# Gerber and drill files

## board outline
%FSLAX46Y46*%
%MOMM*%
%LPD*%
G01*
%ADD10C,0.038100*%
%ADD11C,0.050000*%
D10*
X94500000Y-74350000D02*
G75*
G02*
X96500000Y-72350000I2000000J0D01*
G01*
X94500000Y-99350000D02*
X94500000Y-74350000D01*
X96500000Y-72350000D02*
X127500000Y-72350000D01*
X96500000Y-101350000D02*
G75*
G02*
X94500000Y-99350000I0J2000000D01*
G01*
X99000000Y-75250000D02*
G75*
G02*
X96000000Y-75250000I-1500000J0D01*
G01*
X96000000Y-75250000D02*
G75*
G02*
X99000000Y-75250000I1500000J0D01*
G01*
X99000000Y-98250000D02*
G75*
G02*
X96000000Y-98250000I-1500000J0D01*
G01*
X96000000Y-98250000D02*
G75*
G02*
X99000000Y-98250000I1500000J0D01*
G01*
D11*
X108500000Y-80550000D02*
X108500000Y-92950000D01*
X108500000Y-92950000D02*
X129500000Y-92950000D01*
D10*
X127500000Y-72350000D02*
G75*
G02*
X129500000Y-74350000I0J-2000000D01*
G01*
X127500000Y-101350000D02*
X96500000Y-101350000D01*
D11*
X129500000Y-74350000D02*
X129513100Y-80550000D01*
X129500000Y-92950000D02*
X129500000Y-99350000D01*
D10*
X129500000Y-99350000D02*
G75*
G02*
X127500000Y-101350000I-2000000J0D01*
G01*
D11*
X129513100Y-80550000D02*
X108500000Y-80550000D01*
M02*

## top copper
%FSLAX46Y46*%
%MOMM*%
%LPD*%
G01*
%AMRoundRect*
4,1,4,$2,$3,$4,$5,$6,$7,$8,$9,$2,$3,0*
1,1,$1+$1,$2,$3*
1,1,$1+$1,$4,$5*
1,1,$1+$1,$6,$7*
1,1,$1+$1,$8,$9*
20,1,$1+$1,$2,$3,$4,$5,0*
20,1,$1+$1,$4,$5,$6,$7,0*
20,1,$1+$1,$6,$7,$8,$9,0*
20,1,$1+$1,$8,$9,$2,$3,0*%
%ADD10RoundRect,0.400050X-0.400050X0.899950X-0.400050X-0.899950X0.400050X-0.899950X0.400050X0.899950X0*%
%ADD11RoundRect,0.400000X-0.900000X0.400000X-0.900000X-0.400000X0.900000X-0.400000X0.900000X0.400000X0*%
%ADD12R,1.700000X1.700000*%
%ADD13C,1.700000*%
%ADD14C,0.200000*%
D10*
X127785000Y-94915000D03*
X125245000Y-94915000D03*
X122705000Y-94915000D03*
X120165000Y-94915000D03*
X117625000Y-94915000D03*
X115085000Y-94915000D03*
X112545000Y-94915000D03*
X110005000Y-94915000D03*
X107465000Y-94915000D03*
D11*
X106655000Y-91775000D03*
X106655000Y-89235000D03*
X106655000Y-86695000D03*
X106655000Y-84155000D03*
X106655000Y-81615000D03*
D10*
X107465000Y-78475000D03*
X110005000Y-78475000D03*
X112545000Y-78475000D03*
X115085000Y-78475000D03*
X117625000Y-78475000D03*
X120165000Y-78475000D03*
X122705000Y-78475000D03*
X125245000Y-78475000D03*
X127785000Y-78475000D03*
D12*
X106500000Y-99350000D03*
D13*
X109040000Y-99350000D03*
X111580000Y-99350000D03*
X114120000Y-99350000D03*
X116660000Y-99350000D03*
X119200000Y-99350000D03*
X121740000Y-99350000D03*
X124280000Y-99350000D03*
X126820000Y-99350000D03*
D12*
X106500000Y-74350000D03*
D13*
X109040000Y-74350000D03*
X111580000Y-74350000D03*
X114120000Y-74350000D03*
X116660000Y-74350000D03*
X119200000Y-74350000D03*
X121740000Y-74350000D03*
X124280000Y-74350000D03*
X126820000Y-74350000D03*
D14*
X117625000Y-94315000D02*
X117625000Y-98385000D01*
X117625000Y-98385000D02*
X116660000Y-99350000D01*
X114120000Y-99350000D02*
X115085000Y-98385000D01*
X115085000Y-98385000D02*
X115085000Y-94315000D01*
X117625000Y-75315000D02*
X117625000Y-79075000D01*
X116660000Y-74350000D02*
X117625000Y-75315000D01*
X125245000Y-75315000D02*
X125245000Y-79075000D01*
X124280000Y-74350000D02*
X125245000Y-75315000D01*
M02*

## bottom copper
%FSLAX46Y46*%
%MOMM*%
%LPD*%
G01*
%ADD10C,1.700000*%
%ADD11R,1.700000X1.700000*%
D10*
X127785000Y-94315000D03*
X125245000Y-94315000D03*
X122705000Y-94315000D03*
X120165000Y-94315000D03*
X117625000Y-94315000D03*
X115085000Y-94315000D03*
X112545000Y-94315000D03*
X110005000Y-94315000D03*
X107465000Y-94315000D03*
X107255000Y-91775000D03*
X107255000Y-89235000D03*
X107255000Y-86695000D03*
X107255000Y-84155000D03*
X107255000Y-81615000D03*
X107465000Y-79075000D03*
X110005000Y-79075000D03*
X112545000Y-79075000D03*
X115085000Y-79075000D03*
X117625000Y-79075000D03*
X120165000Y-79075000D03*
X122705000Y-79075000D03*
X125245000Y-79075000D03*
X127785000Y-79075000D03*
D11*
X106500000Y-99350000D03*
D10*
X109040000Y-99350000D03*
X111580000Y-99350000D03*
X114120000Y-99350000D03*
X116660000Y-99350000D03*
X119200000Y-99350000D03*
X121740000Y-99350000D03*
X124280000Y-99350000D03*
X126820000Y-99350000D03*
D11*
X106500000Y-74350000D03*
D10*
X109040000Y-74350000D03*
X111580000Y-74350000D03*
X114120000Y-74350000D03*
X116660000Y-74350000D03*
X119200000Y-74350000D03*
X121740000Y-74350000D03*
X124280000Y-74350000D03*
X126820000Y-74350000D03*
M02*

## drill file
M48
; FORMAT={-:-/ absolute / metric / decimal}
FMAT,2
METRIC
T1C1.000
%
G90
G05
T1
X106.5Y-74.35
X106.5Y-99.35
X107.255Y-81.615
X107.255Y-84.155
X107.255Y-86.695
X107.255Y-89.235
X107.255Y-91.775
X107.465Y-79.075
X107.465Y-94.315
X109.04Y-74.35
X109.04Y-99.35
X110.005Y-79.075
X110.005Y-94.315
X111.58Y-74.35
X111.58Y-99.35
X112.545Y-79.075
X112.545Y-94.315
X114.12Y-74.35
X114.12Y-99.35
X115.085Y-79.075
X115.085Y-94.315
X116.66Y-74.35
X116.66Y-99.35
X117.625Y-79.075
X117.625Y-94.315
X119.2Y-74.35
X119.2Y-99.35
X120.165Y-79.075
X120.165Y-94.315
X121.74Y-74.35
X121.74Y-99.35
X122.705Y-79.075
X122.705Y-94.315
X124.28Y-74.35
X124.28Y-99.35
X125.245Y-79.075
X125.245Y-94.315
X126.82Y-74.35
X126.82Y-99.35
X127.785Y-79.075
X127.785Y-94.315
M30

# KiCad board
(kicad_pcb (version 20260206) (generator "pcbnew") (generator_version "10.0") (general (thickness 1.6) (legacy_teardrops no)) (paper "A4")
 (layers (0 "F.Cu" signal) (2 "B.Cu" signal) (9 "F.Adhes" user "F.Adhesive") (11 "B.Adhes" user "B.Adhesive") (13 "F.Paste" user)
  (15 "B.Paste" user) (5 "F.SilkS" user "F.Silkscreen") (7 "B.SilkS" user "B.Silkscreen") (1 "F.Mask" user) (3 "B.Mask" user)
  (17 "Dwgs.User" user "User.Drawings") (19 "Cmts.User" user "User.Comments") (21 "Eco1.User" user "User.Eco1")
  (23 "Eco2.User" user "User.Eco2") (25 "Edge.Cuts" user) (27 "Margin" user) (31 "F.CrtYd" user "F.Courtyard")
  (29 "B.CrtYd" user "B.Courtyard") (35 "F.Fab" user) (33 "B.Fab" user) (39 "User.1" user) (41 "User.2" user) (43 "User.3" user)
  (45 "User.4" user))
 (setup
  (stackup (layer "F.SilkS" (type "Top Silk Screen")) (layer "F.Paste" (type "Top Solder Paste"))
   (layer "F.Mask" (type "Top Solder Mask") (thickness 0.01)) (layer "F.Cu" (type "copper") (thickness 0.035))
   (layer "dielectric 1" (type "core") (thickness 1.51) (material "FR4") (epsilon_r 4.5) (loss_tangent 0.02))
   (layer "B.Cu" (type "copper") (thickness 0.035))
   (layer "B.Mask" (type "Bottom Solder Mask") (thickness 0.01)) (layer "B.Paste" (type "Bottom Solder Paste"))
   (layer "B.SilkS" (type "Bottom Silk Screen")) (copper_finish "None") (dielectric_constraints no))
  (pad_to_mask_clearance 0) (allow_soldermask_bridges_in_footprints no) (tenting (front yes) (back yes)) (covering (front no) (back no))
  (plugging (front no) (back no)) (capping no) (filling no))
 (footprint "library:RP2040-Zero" (layer "F.Cu") (at 104.925 76.535 -90)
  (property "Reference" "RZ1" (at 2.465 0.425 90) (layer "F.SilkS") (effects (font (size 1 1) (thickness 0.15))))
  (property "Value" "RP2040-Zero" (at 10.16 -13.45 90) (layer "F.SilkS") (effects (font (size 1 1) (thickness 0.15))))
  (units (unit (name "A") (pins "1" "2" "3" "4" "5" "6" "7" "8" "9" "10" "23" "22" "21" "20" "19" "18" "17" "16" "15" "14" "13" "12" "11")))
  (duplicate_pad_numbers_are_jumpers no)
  (pad "1" thru_hole roundrect (at 17.78 -22.86 270) (size 2.6 1.6002) (drill 1 (offset 0.6 0)) (layers "*.Cu" "*.Mask")
   (remove_unused_layers no) (roundrect_rratio 0.25) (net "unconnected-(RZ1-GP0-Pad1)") (thermal_bridge_angle 45)
   (padstack (mode front_inner_back)
    (layer "Inner" (shape roundrect) (size 2.6 1.6002) (offset 0.6 0) (roundrect_rratio 0.25) (zone_connect -1))
    (layer "B.Cu" (shape circle) (size 1.7 1.7))))
  (pad "2" thru_hole roundrect (at 17.78 -20.32 270) (size 2.6 1.6002) (drill 1 (offset 0.6 0)) (layers "*.Cu" "*.Mask")
   (remove_unused_layers no) (roundrect_rratio 0.25) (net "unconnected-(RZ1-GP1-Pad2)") (thermal_bridge_angle 45)
   (padstack (mode front_inner_back)
    (layer "Inner" (shape roundrect) (size 2.6 1.6002) (offset 0.6 0) (roundrect_rratio 0.25) (zone_connect -1))
    (layer "B.Cu" (shape circle) (size 1.7 1.7))))
  (pad "3" thru_hole roundrect (at 17.78 -17.78 270) (size 2.6 1.6002) (drill 1 (offset 0.6 0)) (layers "*.Cu" "*.Mask")
   (remove_unused_layers no) (roundrect_rratio 0.25) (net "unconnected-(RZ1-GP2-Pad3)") (thermal_bridge_angle 45)
   (padstack (mode front_inner_back)
    (layer "Inner" (shape roundrect) (size 2.6 1.6002) (offset 0.6 0) (roundrect_rratio 0.25) (zone_connect -1))
    (layer "B.Cu" (shape circle) (size 1.7 1.7))))
  (pad "4" thru_hole roundrect (at 17.78 -15.24 270) (size 2.6 1.6002) (drill 1 (offset 0.6 0)) (layers "*.Cu" "*.Mask")
   (remove_unused_layers no) (roundrect_rratio 0.25) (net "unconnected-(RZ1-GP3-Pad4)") (thermal_bridge_angle 45)
   (padstack (mode front_inner_back)
    (layer "Inner" (shape roundrect) (size 2.6 1.6002) (offset 0.6 0) (roundrect_rratio 0.25) (zone_connect -1))
    (layer "B.Cu" (shape circle) (size 1.7 1.7))))
  (pad "5" thru_hole roundrect (at 17.78 -12.7 270) (size 2.6 1.6002) (drill 1 (offset 0.6 0)) (layers "*.Cu" "*.Mask")
   (remove_unused_layers no) (roundrect_rratio 0.25) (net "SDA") (thermal_bridge_angle 45)
   (padstack (mode front_inner_back)
    (layer "Inner" (shape roundrect) (size 2.6 1.6002) (offset 0.6 0) (roundrect_rratio 0.25) (zone_connect -1))
    (layer "B.Cu" (shape circle) (size 1.7 1.7))))
  (pad "6" thru_hole roundrect (at 17.78 -10.16 270) (size 2.6 1.6002) (drill 1 (offset 0.6 0)) (layers "*.Cu" "*.Mask")
   (remove_unused_layers no) (roundrect_rratio 0.25) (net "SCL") (thermal_bridge_angle 45)
   (padstack (mode front_inner_back)
    (layer "Inner" (shape roundrect) (size 2.6 1.6002) (offset 0.6 0) (roundrect_rratio 0.25) (zone_connect -1))
    (layer "B.Cu" (shape circle) (size 1.7 1.7))))
  (pad "7" thru_hole roundrect (at 17.78 -7.62 270) (size 2.6 1.6002) (drill 1 (offset 0.6 0)) (layers "*.Cu" "*.Mask")
   (remove_unused_layers no) (roundrect_rratio 0.25) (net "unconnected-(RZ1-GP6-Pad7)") (thermal_bridge_angle 45)
   (padstack (mode front_inner_back)
    (layer "Inner" (shape roundrect) (size 2.6 1.6002) (offset 0.6 0) (roundrect_rratio 0.25) (zone_connect -1))
    (layer "B.Cu" (shape circle) (size 1.7 1.7))))
  (pad "8" thru_hole roundrect (at 17.78 -5.08 270) (size 2.6 1.6002) (drill 1 (offset 0.6 0)) (layers "*.Cu" "*.Mask")
   (remove_unused_layers no) (roundrect_rratio 0.25) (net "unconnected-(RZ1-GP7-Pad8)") (thermal_bridge_angle 45)
   (padstack (mode front_inner_back)
    (layer "Inner" (shape roundrect) (size 2.6 1.6002) (offset 0.6 0) (roundrect_rratio 0.25) (zone_connect -1))
    (layer "B.Cu" (shape circle) (size 1.7 1.7))))
  (pad "9" thru_hole roundrect (at 17.78 -2.54 270) (size 2.6 1.6002) (drill 1 (offset 0.6 0)) (layers "*.Cu" "*.Mask")
   (remove_unused_layers no) (roundrect_rratio 0.25) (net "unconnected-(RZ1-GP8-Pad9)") (thermal_bridge_angle 45)
   (padstack (mode front_inner_back)
    (layer "Inner" (shape roundrect) (size 2.6 1.6002) (offset 0.6 0) (roundrect_rratio 0.25) (zone_connect -1))
    (layer "B.Cu" (shape circle) (size 1.7 1.7))))
  (pad "10" thru_hole roundrect (at 15.24 -2.33 270) (size 1.6 2.6) (drill 1 (offset 0 0.6)) (layers "*.Cu" "*.Mask")
   (remove_unused_layers no) (roundrect_rratio 0.25) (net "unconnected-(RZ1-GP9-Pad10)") (thermal_bridge_angle 45)
   (padstack (mode front_inner_back)
    (layer "Inner" (shape roundrect) (size 1.6 2.6) (offset 0 0.6) (roundrect_rratio 0.25) (zone_connect -1))
    (layer "B.Cu" (shape circle) (size 1.7 1.7))))
  (pad "11" thru_hole roundrect (at 12.7 -2.33 270) (size 1.6 2.6) (drill 1 (offset 0 0.6)) (layers "*.Cu" "*.Mask")
   (remove_unused_layers no) (roundrect_rratio 0.25) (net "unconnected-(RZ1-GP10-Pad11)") (thermal_bridge_angle 45)
   (padstack (mode front_inner_back)
    (layer "Inner" (shape roundrect) (size 1.6 2.6) (offset 0 0.6) (roundrect_rratio 0.25) (zone_connect -1))
    (layer "B.Cu" (shape circle) (size 1.7 1.7))))
  (pad "12" thru_hole roundrect (at 10.16 -2.33 270) (size 1.6 2.6) (drill 1 (offset 0 0.6)) (layers "*.Cu" "*.Mask")
   (remove_unused_layers no) (roundrect_rratio 0.25) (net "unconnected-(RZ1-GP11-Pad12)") (thermal_bridge_angle 45)
   (padstack (mode front_inner_back)
    (layer "Inner" (shape roundrect) (size 1.6 2.6) (offset 0 0.6) (roundrect_rratio 0.25) (zone_connect -1))
    (layer "B.Cu" (shape circle) (size 1.7 1.7))))
  (pad "13" thru_hole roundrect (at 7.62 -2.33 270) (size 1.6 2.6) (drill 1 (offset 0 0.6)) (layers "*.Cu" "*.Mask")
   (remove_unused_layers no) (roundrect_rratio 0.25) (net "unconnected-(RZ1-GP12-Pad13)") (thermal_bridge_angle 45)
   (padstack (mode front_inner_back)
    (layer "Inner" (shape roundrect) (size 1.6 2.6) (offset 0 0.6) (roundrect_rratio 0.25) (zone_connect -1))
    (layer "B.Cu" (shape circle) (size 1.7 1.7))))
  (pad "14" thru_hole roundrect (at 5.08 -2.33 270) (size 1.6 2.6) (drill 1 (offset 0 0.6)) (layers "*.Cu" "*.Mask")
   (remove_unused_layers no) (roundrect_rratio 0.25) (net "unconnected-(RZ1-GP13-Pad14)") (thermal_bridge_angle 45)
   (padstack (mode front_inner_back)
    (layer "Inner" (shape roundrect) (size 1.6 2.6) (offset 0 0.6) (roundrect_rratio 0.25) (zone_connect -1))
    (layer "B.Cu" (shape circle) (size 1.7 1.7))))
  (pad "15" thru_hole roundrect (at 2.54 -2.54 270) (size 2.6 1.6002) (drill 1 (offset -0.6 0)) (layers "*.Cu" "*.Mask")
   (remove_unused_layers no) (roundrect_rratio 0.25) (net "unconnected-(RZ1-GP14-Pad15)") (thermal_bridge_angle 45)
   (padstack (mode front_inner_back)
    (layer "Inner" (shape circle) (size 1.2 1.2) (zone_connect -1)) (layer "B.Cu" (shape circle) (size 1.7 1.7))))
  (pad "16" thru_hole roundrect (at 2.54 -5.08 270) (size 2.6 1.6002) (drill 1 (offset -0.6 0)) (layers "*.Cu" "*.Mask")
   (remove_unused_layers no) (roundrect_rratio 0.25) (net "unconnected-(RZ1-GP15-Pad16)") (thermal_bridge_angle 45)
   (padstack (mode front_inner_back)
    (layer "Inner" (shape circle) (size 1.2 1.2) (zone_connect -1)) (layer "B.Cu" (shape circle) (size 1.7 1.7))))
  (pad "17" thru_hole roundrect (at 2.54 -7.62 270) (size 2.6 1.6002) (drill 1 (offset -0.6 0)) (layers "*.Cu" "*.Mask")
   (remove_unused_layers no) (roundrect_rratio 0.25) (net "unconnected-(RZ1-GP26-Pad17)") (thermal_bridge_angle 45)
   (padstack (mode front_inner_back)
    (layer "Inner" (shape circle) (size 1.2 1.2) (zone_connect -1)) (layer "B.Cu" (shape circle) (size 1.7 1.7))))
  (pad "18" thru_hole roundrect (at 2.54 -10.16 270) (size 2.6 1.6002) (drill 1 (offset -0.6 0)) (layers "*.Cu" "*.Mask")
   (remove_unused_layers no) (roundrect_rratio 0.25) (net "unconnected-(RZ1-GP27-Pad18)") (thermal_bridge_angle 45)
   (padstack (mode front_inner_back)
    (layer "Inner" (shape circle) (size 1.2 1.2) (zone_connect -1)) (layer "B.Cu" (shape circle) (size 1.7 1.7))))
  (pad "19" thru_hole roundrect (at 2.54 -12.7 270) (size 2.6 1.6002) (drill 1 (offset -0.6 0)) (layers "*.Cu" "*.Mask")
   (remove_unused_layers no) (roundrect_rratio 0.25) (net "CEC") (thermal_bridge_angle 45)
   (padstack (mode front_inner_back)
    (layer "Inner" (shape circle) (size 1.2 1.2) (zone_connect -1)) (layer "B.Cu" (shape circle) (size 1.7 1.7))))
  (pad "20" thru_hole roundrect (at 2.54 -15.24 270) (size 2.6 1.6002) (drill 1 (offset -0.6 0)) (layers "*.Cu" "*.Mask")
   (remove_unused_layers no) (roundrect_rratio 0.25) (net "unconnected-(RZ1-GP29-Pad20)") (thermal_bridge_angle 45)
   (padstack (mode front_inner_back)
    (layer "Inner" (shape circle) (size 1.2 1.2) (zone_connect -1)) (layer "B.Cu" (shape circle) (size 1.7 1.7))))
  (pad "21" thru_hole roundrect (at 2.54 -17.78 270) (size 2.6 1.6002) (drill 1 (offset -0.6 0)) (layers "*.Cu" "*.Mask")
   (remove_unused_layers no) (roundrect_rratio 0.25) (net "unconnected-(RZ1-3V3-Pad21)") (thermal_bridge_angle 45)
   (padstack (mode front_inner_back)
    (layer "Inner" (shape circle) (size 1.2 1.2) (zone_connect -1)) (layer "B.Cu" (shape circle) (size 1.7 1.7))))
  (pad "22" thru_hole roundrect (at 2.54 -20.32 270) (size 2.6 1.6002) (drill 1 (offset -0.6 0)) (layers "*.Cu" "*.Mask")
   (remove_unused_layers no) (roundrect_rratio 0.25) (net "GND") (thermal_bridge_angle 45)
   (padstack (mode front_inner_back)
    (layer "Inner" (shape circle) (size 1.2 1.2) (zone_connect -1)) (layer "B.Cu" (shape circle) (size 1.7 1.7))))
  (pad "23" thru_hole roundrect (at 2.54 -22.86 270) (size 2.6 1.6002) (drill 1 (offset -0.6 0)) (layers "*.Cu" "*.Mask")
   (remove_unused_layers no) (roundrect_rratio 0.25) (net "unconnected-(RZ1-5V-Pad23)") (thermal_bridge_angle 45)
   (padstack (mode front_inner_back)
    (layer "Inner" (shape circle) (size 1.2 1.2) (zone_connect -1)) (layer "B.Cu" (shape circle) (size 1.7 1.7)))))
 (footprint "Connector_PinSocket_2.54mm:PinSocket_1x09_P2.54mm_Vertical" (layer "B.Cu") (at 106.5 99.35 -90)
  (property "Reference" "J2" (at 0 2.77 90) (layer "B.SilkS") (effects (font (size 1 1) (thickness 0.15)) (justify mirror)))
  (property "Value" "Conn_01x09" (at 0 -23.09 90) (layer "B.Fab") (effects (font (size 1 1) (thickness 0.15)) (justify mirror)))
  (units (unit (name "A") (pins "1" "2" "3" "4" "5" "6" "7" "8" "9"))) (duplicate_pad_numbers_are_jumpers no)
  (pad "1" thru_hole rect (at 0 0 270) (size 1.7 1.7) (drill 1) (layers "*.Cu" "*.Mask") (remove_unused_layers no)
   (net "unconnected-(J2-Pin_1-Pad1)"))
  (pad "2" thru_hole circle (at 0 -2.54 270) (size 1.7 1.7) (drill 1) (layers "*.Cu" "*.Mask") (remove_unused_layers no)
   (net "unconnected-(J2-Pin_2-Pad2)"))
  (pad "3" thru_hole circle (at 0 -5.08 270) (size 1.7 1.7) (drill 1) (layers "*.Cu" "*.Mask") (remove_unused_layers no)
   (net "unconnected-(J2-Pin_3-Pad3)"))
  (pad "4" thru_hole circle (at 0 -7.62 270) (size 1.7 1.7) (drill 1) (layers "*.Cu" "*.Mask") (remove_unused_layers no) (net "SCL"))
  (pad "5" thru_hole circle (at 0 -10.16 270) (size 1.7 1.7) (drill 1) (layers "*.Cu" "*.Mask") (remove_unused_layers no) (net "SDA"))
  (pad "6" thru_hole circle (at 0 -12.7 270) (size 1.7 1.7) (drill 1) (layers "*.Cu" "*.Mask") (remove_unused_layers no)
   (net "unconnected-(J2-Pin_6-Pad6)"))
  (pad "7" thru_hole circle (at 0 -15.24 270) (size 1.7 1.7) (drill 1) (layers "*.Cu" "*.Mask") (remove_unused_layers no)
   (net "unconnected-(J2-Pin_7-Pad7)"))
  (pad "8" thru_hole circle (at 0 -17.78 270) (size 1.7 1.7) (drill 1) (layers "*.Cu" "*.Mask") (remove_unused_layers no)
   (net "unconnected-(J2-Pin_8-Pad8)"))
  (pad "9" thru_hole circle (at 0 -20.32 270) (size 1.7 1.7) (drill 1) (layers "*.Cu" "*.Mask") (remove_unused_layers no)
   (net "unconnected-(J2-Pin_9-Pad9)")))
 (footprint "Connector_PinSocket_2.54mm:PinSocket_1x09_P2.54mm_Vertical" (layer "B.Cu") (at 106.5 74.35 -90)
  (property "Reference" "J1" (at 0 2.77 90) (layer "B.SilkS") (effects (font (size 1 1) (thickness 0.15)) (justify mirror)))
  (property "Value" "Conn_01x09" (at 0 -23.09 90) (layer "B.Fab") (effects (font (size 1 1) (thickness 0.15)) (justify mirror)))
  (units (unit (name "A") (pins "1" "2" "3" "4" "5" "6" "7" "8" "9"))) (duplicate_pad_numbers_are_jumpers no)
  (pad "1" thru_hole rect (at 0 0 270) (size 1.7 1.7) (drill 1) (layers "*.Cu" "*.Mask") (remove_unused_layers no)
   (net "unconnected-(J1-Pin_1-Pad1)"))
  (pad "2" thru_hole circle (at 0 -2.54 270) (size 1.7 1.7) (drill 1) (layers "*.Cu" "*.Mask") (remove_unused_layers no)
   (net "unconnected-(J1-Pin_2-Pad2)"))
  (pad "3" thru_hole circle (at 0 -5.08 270) (size 1.7 1.7) (drill 1) (layers "*.Cu" "*.Mask") (remove_unused_layers no)
   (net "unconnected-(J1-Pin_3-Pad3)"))
  (pad "4" thru_hole circle (at 0 -7.62 270) (size 1.7 1.7) (drill 1) (layers "*.Cu" "*.Mask") (remove_unused_layers no)
   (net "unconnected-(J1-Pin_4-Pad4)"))
  (pad "5" thru_hole circle (at 0 -10.16 270) (size 1.7 1.7) (drill 1) (layers "*.Cu" "*.Mask") (remove_unused_layers no) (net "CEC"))
  (pad "6" thru_hole circle (at 0 -12.7 270) (size 1.7 1.7) (drill 1) (layers "*.Cu" "*.Mask") (remove_unused_layers no)
   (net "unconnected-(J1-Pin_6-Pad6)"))
  (pad "7" thru_hole circle (at 0 -15.24 270) (size 1.7 1.7) (drill 1) (layers "*.Cu" "*.Mask") (remove_unused_layers no)
   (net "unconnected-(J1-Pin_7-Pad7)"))
  (pad "8" thru_hole circle (at 0 -17.78 270) (size 1.7 1.7) (drill 1) (layers "*.Cu" "*.Mask") (remove_unused_layers no) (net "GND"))
  (pad "9" thru_hole circle (at 0 -20.32 270) (size 1.7 1.7) (drill 1) (layers "*.Cu" "*.Mask") (remove_unused_layers no)
   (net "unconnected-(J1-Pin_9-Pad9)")))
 (gr_arc (start 94.5 74.35) (mid 95.085786 72.935786) (end 96.5 72.35) (stroke (width 0.0381) (type default)) (layer "Edge.Cuts"))
 (gr_line (start 94.5 99.35) (end 94.5 74.35) (stroke (width 0.0381) (type default)) (layer "Edge.Cuts"))
 (gr_line (start 96.5 72.35) (end 127.5 72.35) (stroke (width 0.0381) (type default)) (layer "Edge.Cuts"))
 (gr_arc (start 96.5 101.35) (mid 95.085786 100.764214) (end 94.5 99.35) (stroke (width 0.0381) (type default)) (layer "Edge.Cuts"))
 (gr_circle (center 97.5 75.25) (end 99 75.25) (stroke (width 0.0381) (type default)) (fill no) (layer "Edge.Cuts"))
 (gr_circle (center 97.5 98.25) (end 99 98.25) (stroke (width 0.0381) (type default)) (fill no) (layer "Edge.Cuts"))
 (gr_line (start 108.5 80.55) (end 108.5 92.95) (stroke (width 0.05) (type default)) (layer "Edge.Cuts"))
 (gr_line (start 108.5 92.95) (end 129.5 92.95) (stroke (width 0.05) (type default)) (layer "Edge.Cuts"))
 (gr_arc (start 127.5 72.35) (mid 128.914214 72.935786) (end 129.5 74.35) (stroke (width 0.0381) (type default)) (layer "Edge.Cuts"))
 (gr_line (start 127.5 101.35) (end 96.5 101.35) (stroke (width 0.0381) (type default)) (layer "Edge.Cuts"))
 (gr_line (start 129.5 74.35) (end 129.5131 80.55) (stroke (width 0.05) (type default)) (layer "Edge.Cuts"))
 (gr_line (start 129.5 92.95) (end 129.5 99.35) (stroke (width 0.05) (type default)) (layer "Edge.Cuts"))
 (gr_arc (start 129.5 99.35) (mid 128.914214 100.764214) (end 127.5 101.35) (stroke (width 0.0381) (type default)) (layer "Edge.Cuts"))
 (gr_line (start 129.5131 80.55) (end 108.5 80.55) (stroke (width 0.05) (type default)) (layer "Edge.Cuts"))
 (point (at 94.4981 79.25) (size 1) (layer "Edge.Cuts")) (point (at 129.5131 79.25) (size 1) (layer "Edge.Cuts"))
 (segment (start 117.625 94.315) (end 117.625 98.385) (width 0.2) (layer "F.Cu") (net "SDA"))
 (segment (start 117.625 98.385) (end 116.66 99.35) (width 0.2) (layer "F.Cu") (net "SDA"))
 (segment (start 114.12 99.35) (end 115.085 98.385) (width 0.2) (layer "F.Cu") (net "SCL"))
 (segment (start 115.085 98.385) (end 115.085 94.315) (width 0.2) (layer "F.Cu") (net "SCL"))
 (segment (start 117.625 75.315) (end 117.625 79.075) (width 0.2) (layer "F.Cu") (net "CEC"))
 (segment (start 116.66 74.35) (end 117.625 75.315) (width 0.2) (layer "F.Cu") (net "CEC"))
 (segment (start 125.245 75.315) (end 125.245 79.075) (width 0.2) (layer "F.Cu") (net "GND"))
 (segment (start 124.28 74.35) (end 125.245 75.315) (width 0.2) (layer "F.Cu") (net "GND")))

